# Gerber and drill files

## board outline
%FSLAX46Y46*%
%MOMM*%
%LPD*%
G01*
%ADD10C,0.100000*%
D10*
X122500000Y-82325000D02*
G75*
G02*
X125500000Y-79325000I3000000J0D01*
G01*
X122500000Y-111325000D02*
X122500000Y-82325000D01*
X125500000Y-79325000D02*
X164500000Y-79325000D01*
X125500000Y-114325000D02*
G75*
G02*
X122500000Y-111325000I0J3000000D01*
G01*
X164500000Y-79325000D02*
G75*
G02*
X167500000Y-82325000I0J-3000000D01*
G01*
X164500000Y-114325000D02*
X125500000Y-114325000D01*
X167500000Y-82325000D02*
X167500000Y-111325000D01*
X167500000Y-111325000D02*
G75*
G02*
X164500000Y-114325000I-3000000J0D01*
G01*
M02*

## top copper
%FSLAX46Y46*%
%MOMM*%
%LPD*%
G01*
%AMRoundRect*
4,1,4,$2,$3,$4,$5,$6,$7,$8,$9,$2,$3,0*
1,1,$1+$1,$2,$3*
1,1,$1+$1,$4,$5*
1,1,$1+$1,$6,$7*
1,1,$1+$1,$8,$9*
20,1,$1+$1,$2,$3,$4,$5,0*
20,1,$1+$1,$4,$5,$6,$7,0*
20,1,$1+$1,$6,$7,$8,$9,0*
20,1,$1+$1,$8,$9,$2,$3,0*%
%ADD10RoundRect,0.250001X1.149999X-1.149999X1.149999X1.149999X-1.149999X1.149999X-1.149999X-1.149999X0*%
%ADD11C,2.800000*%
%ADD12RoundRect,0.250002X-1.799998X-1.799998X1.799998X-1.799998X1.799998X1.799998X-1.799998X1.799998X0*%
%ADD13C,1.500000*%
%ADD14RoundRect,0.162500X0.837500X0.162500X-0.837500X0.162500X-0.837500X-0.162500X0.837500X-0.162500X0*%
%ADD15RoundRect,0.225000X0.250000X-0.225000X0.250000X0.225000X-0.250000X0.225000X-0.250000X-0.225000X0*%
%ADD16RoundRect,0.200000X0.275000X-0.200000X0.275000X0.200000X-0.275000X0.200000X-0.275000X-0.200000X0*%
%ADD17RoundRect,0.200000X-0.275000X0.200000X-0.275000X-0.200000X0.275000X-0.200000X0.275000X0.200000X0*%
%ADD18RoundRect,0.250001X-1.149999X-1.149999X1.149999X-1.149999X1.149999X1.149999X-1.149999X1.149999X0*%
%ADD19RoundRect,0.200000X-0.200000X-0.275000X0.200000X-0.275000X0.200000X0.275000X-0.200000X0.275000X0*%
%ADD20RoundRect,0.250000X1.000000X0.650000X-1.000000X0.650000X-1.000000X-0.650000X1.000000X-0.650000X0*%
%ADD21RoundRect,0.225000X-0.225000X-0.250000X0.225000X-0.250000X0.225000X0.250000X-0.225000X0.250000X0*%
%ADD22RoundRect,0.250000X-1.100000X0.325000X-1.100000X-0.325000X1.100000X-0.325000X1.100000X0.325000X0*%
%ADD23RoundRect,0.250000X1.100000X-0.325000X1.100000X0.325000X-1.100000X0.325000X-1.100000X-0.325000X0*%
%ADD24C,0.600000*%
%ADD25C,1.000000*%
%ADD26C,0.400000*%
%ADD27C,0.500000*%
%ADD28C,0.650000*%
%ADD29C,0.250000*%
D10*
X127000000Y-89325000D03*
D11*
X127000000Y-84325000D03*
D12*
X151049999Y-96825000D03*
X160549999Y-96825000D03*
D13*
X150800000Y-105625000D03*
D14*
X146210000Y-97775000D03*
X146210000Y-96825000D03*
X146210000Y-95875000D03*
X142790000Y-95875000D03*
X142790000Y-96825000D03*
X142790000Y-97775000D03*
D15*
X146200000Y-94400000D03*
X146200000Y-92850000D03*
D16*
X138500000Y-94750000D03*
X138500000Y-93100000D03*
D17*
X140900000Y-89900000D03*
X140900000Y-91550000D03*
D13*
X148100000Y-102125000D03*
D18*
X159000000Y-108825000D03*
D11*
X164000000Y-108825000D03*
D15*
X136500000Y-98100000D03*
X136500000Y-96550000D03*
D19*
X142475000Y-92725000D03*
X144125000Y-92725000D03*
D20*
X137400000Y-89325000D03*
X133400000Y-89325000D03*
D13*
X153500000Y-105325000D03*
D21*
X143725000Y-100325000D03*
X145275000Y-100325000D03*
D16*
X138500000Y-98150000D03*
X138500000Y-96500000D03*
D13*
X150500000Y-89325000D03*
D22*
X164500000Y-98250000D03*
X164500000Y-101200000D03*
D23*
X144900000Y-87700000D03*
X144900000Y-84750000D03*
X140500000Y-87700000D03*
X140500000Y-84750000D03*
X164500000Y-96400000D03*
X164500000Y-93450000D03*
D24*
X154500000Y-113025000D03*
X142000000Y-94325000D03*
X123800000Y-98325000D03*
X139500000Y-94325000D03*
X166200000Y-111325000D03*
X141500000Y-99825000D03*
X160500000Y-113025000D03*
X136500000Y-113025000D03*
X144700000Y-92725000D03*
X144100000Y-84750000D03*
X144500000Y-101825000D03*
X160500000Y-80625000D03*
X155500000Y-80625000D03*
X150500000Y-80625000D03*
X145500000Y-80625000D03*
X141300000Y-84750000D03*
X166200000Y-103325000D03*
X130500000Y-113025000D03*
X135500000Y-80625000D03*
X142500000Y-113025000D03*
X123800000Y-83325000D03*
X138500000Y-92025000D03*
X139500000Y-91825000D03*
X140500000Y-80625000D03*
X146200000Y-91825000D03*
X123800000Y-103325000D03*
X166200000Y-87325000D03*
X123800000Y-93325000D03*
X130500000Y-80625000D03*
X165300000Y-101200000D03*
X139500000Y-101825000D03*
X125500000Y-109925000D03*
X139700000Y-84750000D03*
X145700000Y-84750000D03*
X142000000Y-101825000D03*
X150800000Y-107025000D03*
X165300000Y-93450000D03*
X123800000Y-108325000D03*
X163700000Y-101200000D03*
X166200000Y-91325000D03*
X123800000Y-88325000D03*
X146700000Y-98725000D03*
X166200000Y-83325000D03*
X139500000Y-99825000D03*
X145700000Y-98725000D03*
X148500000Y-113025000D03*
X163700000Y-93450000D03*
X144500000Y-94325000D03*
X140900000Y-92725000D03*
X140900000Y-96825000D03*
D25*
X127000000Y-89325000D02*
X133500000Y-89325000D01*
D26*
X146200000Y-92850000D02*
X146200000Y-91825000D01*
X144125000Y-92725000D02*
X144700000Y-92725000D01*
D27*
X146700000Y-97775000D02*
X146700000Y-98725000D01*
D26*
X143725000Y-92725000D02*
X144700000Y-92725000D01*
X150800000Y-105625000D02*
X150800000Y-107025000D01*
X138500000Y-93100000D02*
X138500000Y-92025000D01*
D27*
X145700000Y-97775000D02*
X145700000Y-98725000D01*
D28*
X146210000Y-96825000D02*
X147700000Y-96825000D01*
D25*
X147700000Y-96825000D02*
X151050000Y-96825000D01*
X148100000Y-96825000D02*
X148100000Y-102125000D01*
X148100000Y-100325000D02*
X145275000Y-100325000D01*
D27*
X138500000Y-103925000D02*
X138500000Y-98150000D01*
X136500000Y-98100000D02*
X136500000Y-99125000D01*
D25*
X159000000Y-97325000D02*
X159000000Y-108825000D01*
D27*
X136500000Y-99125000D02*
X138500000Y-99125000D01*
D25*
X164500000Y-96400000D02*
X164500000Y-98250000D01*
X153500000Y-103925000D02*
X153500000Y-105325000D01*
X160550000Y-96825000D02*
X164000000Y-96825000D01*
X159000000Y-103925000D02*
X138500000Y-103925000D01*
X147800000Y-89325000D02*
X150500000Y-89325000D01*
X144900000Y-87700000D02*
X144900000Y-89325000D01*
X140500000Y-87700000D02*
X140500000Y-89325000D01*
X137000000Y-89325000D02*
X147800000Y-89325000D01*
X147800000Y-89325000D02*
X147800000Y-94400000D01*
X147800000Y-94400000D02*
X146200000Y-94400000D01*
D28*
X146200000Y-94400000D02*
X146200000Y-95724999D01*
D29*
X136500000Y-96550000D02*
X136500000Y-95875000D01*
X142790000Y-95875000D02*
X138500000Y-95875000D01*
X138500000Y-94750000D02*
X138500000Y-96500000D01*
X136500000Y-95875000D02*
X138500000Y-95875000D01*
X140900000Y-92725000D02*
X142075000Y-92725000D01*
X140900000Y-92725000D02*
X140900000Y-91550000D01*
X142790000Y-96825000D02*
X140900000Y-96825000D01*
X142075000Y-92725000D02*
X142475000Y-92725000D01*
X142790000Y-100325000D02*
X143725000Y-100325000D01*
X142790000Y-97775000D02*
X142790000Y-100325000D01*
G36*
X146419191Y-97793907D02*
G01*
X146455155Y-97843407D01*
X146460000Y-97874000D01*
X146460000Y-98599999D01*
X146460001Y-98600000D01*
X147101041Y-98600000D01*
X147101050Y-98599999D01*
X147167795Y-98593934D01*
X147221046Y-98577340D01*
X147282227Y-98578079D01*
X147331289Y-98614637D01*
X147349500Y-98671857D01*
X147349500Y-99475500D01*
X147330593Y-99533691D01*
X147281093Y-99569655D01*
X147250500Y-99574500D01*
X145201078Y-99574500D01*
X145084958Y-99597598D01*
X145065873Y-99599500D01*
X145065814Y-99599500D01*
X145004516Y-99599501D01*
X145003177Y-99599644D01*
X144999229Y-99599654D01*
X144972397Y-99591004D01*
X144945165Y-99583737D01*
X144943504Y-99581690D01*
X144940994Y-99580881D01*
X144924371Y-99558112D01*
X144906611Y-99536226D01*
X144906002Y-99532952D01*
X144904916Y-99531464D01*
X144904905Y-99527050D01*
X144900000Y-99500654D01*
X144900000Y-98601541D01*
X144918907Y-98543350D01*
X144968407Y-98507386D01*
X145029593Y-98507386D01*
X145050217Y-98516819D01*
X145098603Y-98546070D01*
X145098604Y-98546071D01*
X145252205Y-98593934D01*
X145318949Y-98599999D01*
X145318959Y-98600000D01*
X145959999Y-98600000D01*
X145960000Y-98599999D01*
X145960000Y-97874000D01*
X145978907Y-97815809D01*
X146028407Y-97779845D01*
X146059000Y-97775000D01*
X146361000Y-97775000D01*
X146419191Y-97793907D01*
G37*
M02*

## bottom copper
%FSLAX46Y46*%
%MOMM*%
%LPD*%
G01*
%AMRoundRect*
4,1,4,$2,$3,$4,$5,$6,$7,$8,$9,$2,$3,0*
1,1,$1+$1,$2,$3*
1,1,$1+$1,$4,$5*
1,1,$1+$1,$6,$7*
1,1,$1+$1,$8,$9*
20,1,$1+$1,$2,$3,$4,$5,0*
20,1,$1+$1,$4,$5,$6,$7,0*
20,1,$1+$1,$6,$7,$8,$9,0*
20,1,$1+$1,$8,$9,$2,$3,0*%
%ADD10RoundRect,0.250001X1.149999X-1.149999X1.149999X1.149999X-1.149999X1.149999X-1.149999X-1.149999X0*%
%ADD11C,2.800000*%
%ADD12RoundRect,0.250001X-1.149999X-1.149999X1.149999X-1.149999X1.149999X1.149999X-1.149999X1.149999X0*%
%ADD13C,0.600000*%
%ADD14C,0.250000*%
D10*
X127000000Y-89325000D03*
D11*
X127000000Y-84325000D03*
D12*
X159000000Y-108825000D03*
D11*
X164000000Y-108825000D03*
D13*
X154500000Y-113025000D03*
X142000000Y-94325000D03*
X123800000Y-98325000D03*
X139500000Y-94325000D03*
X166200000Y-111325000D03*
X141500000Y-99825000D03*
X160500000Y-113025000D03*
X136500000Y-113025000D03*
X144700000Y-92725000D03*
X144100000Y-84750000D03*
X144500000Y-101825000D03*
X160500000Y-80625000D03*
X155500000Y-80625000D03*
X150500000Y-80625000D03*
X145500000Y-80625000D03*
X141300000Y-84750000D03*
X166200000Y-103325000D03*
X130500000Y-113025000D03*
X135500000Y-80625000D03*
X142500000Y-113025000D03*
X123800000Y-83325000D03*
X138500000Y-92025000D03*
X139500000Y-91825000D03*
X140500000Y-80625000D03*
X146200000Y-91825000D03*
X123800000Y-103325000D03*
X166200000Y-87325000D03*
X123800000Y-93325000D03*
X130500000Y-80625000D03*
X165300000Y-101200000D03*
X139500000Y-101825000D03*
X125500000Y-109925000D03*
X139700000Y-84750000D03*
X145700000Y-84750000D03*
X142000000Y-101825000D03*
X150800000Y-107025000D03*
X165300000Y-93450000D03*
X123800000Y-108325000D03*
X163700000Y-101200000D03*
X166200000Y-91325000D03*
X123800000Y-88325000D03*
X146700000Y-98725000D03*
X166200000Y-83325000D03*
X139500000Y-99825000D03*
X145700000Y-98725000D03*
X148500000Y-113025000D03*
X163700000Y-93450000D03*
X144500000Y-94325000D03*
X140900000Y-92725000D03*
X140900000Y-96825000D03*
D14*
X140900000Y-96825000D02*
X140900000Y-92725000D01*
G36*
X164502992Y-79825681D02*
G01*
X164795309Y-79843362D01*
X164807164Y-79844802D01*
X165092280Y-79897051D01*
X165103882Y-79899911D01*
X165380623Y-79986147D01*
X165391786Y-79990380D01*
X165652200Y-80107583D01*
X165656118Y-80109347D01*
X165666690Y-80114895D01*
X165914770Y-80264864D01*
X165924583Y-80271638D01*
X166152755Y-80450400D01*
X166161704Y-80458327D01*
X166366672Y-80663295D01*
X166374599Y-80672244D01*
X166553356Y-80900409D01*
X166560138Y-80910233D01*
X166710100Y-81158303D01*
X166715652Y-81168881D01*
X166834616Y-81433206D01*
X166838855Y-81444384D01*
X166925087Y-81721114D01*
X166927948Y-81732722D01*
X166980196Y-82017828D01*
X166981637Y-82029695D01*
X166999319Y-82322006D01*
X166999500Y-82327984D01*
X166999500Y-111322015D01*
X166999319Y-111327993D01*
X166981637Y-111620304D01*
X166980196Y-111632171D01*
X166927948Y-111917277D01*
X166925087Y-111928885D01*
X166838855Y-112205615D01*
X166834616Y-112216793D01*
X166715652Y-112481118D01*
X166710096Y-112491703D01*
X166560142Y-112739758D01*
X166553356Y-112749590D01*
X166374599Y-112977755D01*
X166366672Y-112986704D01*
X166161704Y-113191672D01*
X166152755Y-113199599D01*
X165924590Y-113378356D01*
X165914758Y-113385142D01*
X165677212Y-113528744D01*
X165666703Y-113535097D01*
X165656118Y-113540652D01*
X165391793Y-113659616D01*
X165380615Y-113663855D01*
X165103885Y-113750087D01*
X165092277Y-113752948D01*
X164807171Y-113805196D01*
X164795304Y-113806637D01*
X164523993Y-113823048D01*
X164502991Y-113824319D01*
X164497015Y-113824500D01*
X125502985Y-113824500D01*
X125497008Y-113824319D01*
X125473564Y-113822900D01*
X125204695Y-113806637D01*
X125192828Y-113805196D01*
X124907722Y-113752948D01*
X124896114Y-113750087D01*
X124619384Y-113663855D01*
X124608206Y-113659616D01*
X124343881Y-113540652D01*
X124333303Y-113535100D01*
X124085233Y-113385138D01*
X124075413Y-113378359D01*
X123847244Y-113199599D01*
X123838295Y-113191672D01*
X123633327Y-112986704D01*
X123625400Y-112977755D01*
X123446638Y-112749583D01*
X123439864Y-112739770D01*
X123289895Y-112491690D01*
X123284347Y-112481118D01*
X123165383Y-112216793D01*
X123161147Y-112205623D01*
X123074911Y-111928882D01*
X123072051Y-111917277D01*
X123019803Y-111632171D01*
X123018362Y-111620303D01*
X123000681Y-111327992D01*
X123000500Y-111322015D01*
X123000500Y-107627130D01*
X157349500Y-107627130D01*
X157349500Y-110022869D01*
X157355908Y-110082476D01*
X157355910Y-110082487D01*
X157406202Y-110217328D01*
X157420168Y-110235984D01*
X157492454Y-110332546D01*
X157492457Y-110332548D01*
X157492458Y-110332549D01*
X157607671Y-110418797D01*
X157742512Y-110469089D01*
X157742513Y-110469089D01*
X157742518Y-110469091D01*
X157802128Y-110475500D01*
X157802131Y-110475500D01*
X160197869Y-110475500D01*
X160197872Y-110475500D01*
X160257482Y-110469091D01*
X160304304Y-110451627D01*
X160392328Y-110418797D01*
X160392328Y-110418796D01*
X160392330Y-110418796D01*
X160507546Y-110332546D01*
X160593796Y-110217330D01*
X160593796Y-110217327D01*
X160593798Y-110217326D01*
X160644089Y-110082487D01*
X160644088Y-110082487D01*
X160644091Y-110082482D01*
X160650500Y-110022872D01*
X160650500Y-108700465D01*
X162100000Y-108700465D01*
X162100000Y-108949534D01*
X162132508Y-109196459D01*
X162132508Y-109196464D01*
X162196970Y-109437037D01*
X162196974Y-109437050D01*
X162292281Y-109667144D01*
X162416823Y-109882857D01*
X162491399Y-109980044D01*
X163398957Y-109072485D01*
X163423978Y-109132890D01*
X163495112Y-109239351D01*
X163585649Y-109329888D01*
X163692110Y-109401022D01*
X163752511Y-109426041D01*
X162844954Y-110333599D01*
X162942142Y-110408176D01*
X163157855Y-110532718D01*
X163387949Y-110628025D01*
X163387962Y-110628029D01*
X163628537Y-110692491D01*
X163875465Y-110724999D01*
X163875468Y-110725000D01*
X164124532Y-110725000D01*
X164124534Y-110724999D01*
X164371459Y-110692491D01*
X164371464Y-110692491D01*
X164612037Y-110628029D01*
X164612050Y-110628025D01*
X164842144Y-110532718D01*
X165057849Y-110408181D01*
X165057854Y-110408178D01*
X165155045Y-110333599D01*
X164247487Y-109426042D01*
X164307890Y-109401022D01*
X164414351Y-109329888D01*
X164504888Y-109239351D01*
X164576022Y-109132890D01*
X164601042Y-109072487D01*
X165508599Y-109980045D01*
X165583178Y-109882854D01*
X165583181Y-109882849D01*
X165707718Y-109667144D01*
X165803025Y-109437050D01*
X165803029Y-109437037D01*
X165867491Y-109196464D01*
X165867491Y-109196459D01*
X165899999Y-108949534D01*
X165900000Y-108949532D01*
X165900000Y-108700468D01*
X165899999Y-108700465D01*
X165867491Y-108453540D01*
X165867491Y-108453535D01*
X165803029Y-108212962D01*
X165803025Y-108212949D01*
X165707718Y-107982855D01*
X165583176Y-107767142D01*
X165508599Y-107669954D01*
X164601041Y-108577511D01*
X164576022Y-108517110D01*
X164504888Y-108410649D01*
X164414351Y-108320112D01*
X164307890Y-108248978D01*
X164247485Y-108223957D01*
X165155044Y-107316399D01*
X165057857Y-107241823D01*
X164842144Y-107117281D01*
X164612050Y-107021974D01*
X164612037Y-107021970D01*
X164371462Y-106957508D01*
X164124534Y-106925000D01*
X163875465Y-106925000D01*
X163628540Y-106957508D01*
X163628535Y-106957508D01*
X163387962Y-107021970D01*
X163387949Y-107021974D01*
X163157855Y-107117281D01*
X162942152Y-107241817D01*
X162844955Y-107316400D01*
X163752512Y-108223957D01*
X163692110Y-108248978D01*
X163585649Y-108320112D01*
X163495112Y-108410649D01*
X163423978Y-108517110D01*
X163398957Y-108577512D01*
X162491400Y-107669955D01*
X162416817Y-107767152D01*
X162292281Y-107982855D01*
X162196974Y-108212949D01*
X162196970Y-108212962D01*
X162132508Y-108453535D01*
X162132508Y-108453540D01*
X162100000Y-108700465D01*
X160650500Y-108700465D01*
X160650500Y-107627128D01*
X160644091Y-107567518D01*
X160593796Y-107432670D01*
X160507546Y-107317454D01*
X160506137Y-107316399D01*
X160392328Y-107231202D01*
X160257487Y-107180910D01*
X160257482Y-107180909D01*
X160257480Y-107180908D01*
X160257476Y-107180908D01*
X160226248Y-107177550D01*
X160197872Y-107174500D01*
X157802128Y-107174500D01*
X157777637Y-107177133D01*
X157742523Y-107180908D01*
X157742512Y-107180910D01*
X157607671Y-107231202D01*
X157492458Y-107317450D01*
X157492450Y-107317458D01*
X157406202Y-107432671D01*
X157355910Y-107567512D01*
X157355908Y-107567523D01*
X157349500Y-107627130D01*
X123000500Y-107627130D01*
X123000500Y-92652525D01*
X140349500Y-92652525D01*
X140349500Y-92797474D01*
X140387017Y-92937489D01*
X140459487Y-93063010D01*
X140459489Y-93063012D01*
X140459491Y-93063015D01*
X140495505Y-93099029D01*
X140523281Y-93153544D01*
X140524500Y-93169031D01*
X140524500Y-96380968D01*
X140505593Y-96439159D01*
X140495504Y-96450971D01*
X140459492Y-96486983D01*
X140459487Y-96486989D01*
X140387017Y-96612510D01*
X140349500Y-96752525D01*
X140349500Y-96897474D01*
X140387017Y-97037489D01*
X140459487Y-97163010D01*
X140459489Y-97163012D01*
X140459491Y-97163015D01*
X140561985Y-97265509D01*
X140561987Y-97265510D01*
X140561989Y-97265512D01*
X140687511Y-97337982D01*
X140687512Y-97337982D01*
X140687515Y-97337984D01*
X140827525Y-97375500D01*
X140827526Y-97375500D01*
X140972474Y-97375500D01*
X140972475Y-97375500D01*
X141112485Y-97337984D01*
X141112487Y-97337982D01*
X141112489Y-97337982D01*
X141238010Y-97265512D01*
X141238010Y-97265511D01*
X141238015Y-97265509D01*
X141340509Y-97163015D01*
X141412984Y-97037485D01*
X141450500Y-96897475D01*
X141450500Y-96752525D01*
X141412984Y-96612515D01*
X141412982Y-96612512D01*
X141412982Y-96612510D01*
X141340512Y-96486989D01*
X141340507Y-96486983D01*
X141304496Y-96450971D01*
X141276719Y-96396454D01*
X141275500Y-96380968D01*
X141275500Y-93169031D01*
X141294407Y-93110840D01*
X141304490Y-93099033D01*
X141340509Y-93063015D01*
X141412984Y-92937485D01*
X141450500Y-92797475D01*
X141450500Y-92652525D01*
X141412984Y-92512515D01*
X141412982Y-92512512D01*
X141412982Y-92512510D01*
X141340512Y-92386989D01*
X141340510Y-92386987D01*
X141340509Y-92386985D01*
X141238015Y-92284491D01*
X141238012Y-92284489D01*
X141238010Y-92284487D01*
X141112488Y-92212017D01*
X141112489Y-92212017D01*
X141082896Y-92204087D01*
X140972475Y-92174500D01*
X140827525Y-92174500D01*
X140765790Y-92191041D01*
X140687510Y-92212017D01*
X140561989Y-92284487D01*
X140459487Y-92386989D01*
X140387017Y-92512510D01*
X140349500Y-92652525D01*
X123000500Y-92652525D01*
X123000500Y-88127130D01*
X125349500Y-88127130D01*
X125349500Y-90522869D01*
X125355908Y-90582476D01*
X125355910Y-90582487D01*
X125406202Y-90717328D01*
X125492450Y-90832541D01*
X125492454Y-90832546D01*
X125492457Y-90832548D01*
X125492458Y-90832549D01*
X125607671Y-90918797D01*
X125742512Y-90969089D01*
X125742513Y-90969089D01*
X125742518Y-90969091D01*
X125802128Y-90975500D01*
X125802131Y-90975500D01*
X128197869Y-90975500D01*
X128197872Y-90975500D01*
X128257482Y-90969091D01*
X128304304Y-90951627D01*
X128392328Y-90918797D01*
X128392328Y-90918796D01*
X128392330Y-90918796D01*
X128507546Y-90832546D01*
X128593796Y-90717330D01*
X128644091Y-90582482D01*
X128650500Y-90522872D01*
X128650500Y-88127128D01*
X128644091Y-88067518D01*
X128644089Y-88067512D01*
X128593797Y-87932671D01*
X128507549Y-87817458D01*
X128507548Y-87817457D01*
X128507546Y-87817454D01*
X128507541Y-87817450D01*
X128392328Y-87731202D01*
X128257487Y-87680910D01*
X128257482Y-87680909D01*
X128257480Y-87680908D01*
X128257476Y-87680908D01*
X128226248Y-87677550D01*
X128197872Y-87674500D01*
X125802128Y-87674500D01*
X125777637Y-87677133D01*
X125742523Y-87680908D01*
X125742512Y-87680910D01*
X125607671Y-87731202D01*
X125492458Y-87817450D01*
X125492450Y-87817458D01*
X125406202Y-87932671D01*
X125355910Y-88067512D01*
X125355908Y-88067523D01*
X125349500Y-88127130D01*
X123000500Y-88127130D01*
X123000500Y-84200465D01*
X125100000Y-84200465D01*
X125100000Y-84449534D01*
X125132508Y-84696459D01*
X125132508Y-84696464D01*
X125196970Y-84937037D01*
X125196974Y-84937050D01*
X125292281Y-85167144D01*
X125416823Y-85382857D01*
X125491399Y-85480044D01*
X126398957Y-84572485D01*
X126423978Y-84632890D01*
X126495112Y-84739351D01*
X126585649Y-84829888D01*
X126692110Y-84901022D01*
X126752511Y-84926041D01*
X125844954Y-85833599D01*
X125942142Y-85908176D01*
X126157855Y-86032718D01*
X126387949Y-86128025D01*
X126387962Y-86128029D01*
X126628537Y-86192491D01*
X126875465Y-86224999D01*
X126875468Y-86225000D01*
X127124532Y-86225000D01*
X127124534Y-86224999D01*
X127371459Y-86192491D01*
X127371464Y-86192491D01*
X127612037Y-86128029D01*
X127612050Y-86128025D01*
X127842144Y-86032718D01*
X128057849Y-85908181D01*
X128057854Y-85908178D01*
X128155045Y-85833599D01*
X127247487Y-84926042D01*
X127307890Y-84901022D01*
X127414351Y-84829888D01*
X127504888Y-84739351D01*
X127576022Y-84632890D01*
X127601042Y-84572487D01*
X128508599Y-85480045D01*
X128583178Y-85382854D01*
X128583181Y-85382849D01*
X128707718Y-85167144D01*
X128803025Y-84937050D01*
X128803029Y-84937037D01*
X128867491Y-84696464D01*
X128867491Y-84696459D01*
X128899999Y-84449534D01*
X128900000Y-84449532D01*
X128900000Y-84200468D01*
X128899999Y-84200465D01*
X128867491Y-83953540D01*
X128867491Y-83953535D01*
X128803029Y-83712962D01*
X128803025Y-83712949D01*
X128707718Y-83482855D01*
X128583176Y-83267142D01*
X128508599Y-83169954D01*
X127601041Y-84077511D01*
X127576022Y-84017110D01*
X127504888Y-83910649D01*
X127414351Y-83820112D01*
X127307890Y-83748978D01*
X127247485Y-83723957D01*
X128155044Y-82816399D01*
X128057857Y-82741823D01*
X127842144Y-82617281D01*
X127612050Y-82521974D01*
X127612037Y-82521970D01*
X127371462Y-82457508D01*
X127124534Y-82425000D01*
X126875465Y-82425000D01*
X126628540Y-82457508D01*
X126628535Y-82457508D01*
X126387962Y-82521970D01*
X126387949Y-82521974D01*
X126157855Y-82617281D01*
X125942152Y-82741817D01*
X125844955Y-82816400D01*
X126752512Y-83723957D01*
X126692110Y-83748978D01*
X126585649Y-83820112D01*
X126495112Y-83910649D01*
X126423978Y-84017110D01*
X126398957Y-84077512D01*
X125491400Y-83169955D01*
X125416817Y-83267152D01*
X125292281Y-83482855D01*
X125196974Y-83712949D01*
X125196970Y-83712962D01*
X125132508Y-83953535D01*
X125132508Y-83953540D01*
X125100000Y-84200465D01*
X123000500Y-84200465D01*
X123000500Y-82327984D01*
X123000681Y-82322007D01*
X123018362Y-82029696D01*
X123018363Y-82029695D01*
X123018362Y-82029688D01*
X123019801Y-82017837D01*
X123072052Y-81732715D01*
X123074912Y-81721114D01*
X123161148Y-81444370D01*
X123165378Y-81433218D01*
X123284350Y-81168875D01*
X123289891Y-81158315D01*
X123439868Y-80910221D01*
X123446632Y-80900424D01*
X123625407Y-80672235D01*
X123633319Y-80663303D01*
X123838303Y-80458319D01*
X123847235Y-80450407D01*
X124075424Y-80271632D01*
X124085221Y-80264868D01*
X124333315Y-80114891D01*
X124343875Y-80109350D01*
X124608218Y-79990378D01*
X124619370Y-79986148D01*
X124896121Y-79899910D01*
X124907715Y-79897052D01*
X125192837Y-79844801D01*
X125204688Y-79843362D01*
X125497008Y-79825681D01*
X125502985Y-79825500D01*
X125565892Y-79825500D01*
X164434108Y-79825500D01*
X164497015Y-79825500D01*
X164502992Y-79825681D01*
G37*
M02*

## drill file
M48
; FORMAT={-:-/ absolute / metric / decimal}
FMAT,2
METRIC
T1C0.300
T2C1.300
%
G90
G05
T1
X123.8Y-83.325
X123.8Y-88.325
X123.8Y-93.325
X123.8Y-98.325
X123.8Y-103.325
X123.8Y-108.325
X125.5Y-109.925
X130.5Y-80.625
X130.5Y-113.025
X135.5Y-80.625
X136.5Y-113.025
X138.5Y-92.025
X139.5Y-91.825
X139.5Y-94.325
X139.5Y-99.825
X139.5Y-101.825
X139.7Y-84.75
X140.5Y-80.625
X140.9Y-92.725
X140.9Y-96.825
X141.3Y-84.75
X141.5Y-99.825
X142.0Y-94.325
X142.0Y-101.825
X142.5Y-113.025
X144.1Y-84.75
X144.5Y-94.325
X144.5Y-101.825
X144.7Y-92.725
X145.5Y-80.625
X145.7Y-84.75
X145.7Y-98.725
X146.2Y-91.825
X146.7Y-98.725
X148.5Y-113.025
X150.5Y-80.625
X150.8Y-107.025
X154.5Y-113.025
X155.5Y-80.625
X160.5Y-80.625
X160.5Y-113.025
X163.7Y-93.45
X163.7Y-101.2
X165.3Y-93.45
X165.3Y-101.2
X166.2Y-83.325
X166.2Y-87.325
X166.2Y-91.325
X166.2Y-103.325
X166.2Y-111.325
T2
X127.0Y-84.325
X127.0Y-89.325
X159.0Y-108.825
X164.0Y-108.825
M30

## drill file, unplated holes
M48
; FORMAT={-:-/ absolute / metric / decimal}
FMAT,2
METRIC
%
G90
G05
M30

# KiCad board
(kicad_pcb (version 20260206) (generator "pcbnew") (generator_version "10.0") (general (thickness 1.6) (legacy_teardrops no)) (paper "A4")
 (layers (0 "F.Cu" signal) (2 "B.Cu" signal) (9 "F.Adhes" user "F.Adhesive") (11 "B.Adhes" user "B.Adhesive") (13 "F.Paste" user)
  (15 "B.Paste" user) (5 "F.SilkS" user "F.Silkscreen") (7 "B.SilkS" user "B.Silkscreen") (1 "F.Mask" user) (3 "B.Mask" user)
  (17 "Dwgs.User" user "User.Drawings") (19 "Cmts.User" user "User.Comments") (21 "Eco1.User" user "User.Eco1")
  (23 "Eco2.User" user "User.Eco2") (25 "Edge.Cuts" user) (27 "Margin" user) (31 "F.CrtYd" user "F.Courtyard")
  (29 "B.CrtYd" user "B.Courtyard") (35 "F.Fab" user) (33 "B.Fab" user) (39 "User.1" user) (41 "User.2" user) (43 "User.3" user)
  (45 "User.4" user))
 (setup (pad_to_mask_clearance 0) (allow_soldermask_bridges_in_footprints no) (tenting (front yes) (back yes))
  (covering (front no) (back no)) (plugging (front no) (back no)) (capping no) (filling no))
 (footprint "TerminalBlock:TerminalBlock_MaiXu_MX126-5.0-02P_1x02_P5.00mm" (layer "F.Cu") (at 127 89.325 90)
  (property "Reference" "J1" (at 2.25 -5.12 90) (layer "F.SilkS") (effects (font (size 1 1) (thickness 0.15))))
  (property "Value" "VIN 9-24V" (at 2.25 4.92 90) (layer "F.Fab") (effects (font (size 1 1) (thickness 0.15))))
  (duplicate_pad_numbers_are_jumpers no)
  (pad "1" thru_hole roundrect (at 0 0 90) (size 2.8 2.8) (drill 1.3) (layers "*.Cu" "*.Mask") (remove_unused_layers no)
   (roundrect_rratio 0.089286) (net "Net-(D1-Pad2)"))
  (pad "2" thru_hole circle (at 5 0 90) (size 2.8 2.8) (drill 1.3) (layers "*.Cu" "*.Mask") (remove_unused_layers no) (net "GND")))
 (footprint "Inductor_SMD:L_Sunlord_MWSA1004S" (layer "F.Cu") (at 155.799999 96.825)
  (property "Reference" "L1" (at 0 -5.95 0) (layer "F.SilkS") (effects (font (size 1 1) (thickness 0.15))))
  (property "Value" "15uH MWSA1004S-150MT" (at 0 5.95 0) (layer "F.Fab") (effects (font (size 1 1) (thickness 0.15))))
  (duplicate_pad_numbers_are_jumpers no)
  (pad "1" smd roundrect (at -4.75 0) (size 4.1 4.1) (layers "F.Cu" "F.Mask" "F.Paste") (roundrect_rratio 0.060976) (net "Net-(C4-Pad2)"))
  (pad "2" smd roundrect (at 4.75 0) (size 4.1 4.1) (layers "F.Cu" "F.Mask" "F.Paste") (roundrect_rratio 0.060976) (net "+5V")))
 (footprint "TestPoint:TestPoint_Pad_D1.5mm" (layer "F.Cu") (at 150.8 105.625)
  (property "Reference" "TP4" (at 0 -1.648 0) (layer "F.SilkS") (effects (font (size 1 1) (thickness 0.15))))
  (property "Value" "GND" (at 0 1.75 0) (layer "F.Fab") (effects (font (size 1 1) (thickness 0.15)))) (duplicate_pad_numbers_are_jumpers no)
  (pad "1" smd circle (at 0 0) (size 1.5 1.5) (layers "F.Cu" "F.Mask") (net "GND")))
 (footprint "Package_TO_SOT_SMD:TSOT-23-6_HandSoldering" (layer "F.Cu") (at 144.5 96.825 180)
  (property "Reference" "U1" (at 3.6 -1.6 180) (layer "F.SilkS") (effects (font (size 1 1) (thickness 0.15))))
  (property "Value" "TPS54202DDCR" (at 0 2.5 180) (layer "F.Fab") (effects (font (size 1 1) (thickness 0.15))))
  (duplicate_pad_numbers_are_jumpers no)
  (pad "1" smd roundrect (at -1.71 -0.95 180) (size 2 0.65) (layers "F.Cu" "F.Mask" "F.Paste") (roundrect_rratio 0.25) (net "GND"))
  (pad "2" smd roundrect (at -1.71 0 180) (size 2 0.65) (layers "F.Cu" "F.Mask" "F.Paste") (roundrect_rratio 0.25) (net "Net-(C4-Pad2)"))
  (pad "3" smd roundrect (at -1.71 0.95 180) (size 2 0.65) (layers "F.Cu" "F.Mask" "F.Paste") (roundrect_rratio 0.25) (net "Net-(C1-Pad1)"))
  (pad "4" smd roundrect (at 1.71 0.95 180) (size 2 0.65) (layers "F.Cu" "F.Mask" "F.Paste") (roundrect_rratio 0.25) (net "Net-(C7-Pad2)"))
  (pad "5" smd roundrect (at 1.71 0 180) (size 2 0.65) (layers "F.Cu" "F.Mask" "F.Paste") (roundrect_rratio 0.25) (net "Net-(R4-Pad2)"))
  (pad "6" smd roundrect (at 1.71 -0.95 180) (size 2 0.65) (layers "F.Cu" "F.Mask" "F.Paste") (roundrect_rratio 0.25) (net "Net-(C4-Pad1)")))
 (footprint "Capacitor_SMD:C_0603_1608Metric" (layer "F.Cu") (at 146.2 93.625 90)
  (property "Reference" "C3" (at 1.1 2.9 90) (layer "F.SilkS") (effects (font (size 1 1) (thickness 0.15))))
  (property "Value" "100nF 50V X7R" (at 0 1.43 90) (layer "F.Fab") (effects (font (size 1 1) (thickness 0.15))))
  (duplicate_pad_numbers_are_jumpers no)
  (pad "1" smd roundrect (at -0.775 0 90) (size 0.9 0.95) (layers "F.Cu" "F.Mask" "F.Paste") (roundrect_rratio 0.25) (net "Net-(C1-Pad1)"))
  (pad "2" smd roundrect (at 0.775 0 90) (size 0.9 0.95) (layers "F.Cu" "F.Mask" "F.Paste") (roundrect_rratio 0.25) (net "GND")))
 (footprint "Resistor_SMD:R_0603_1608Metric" (layer "F.Cu") (at 138.5 93.925 90)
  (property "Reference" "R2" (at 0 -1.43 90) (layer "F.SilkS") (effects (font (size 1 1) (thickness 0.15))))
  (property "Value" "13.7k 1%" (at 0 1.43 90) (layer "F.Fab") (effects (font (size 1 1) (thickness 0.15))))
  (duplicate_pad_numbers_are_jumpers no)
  (pad "1" smd roundrect (at -0.825 0 90) (size 0.8 0.95) (layers "F.Cu" "F.Mask" "F.Paste") (roundrect_rratio 0.25) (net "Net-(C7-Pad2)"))
  (pad "2" smd roundrect (at 0.825 0 90) (size 0.8 0.95) (layers "F.Cu" "F.Mask" "F.Paste") (roundrect_rratio 0.25) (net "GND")))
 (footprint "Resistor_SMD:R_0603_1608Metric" (layer "F.Cu") (at 140.9 90.725 -90)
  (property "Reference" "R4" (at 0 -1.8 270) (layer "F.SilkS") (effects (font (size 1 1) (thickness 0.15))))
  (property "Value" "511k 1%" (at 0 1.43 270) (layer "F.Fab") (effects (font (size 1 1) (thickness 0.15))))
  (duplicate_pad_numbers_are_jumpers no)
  (pad "1" smd roundrect (at -0.825 0 270) (size 0.8 0.95) (layers "F.Cu" "F.Mask" "F.Paste") (roundrect_rratio 0.25) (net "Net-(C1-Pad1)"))
  (pad "2" smd roundrect (at 0.825 0 270) (size 0.8 0.95) (layers "F.Cu" "F.Mask" "F.Paste") (roundrect_rratio 0.25) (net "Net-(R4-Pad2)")))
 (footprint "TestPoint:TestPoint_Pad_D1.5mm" (layer "F.Cu") (at 148.1 102.125)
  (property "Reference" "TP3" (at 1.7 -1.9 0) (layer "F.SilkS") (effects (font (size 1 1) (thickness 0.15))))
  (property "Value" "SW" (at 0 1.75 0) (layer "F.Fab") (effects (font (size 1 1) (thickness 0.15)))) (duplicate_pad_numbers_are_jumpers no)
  (pad "1" smd circle (at 0 0) (size 1.5 1.5) (layers "F.Cu" "F.Mask") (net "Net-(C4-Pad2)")))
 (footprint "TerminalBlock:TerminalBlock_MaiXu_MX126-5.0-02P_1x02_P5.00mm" (layer "F.Cu") (at 159 108.825)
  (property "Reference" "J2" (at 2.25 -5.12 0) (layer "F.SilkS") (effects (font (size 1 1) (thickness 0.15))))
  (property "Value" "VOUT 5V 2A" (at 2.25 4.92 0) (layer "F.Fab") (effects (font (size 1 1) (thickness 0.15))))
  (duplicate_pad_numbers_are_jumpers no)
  (pad "1" thru_hole roundrect (at 0 0) (size 2.8 2.8) (drill 1.3) (layers "*.Cu" "*.Mask") (remove_unused_layers no)
   (roundrect_rratio 0.089286) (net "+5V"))
  (pad "2" thru_hole circle (at 5 0) (size 2.8 2.8) (drill 1.3) (layers "*.Cu" "*.Mask") (remove_unused_layers no) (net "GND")))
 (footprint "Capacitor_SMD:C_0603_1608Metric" (layer "F.Cu") (at 136.5 97.325 90)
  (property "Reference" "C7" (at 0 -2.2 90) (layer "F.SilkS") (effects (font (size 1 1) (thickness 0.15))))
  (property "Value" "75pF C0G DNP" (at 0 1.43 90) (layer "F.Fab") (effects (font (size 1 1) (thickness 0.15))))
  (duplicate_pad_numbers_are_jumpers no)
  (pad "1" smd roundrect (at -0.775 0 90) (size 0.9 0.95) (layers "F.Cu" "F.Mask" "F.Paste") (roundrect_rratio 0.25) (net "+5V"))
  (pad "2" smd roundrect (at 0.775 0 90) (size 0.9 0.95) (layers "F.Cu" "F.Mask" "F.Paste") (roundrect_rratio 0.25) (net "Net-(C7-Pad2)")))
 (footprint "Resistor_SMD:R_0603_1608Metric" (layer "F.Cu") (at 143.3 92.725)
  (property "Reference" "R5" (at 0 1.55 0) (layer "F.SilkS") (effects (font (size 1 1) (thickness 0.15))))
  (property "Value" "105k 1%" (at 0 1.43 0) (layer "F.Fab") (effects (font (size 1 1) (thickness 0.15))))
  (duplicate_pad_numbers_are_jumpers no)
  (pad "1" smd roundrect (at -0.825 0) (size 0.8 0.95) (layers "F.Cu" "F.Mask" "F.Paste") (roundrect_rratio 0.25) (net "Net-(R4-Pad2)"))
  (pad "2" smd roundrect (at 0.825 0) (size 0.8 0.95) (layers "F.Cu" "F.Mask" "F.Paste") (roundrect_rratio 0.25) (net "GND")))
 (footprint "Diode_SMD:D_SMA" (layer "F.Cu") (at 135.4 89.325 180)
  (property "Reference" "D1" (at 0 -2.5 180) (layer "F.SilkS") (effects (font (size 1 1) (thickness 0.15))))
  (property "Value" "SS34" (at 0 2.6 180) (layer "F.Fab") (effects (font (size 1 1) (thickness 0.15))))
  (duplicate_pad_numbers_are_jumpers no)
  (pad "1" smd roundrect (at -2 0 180) (size 2.5 1.8) (layers "F.Cu" "F.Mask" "F.Paste") (roundrect_rratio 0.1388888889)
   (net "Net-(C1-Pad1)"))
  (pad "2" smd roundrect (at 2 0 180) (size 2.5 1.8) (layers "F.Cu" "F.Mask" "F.Paste") (roundrect_rratio 0.1388888889)
   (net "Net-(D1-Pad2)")))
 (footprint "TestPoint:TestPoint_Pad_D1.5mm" (layer "F.Cu") (at 153.5 105.325)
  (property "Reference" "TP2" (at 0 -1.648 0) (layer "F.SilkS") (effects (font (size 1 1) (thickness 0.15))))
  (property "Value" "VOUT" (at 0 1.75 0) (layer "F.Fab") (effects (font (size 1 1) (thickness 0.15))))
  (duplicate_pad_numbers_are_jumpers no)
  (pad "1" smd circle (at 0 0) (size 1.5 1.5) (layers "F.Cu" "F.Mask") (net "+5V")))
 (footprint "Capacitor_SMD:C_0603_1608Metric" (layer "F.Cu") (at 144.5 100.325)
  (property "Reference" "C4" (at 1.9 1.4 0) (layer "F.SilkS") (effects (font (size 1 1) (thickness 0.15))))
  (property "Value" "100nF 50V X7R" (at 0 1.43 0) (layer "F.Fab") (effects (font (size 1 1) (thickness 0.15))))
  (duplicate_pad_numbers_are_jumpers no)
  (pad "1" smd roundrect (at -0.775 0) (size 0.9 0.95) (layers "F.Cu" "F.Mask" "F.Paste") (roundrect_rratio 0.25) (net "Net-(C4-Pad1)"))
  (pad "2" smd roundrect (at 0.775 0) (size 0.9 0.95) (layers "F.Cu" "F.Mask" "F.Paste") (roundrect_rratio 0.25) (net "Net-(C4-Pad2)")))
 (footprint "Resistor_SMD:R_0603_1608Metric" (layer "F.Cu") (at 138.5 97.325 90)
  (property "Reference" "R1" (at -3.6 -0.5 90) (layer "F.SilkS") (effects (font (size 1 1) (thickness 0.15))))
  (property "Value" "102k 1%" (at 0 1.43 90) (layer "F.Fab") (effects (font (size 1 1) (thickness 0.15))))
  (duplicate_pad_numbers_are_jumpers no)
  (pad "1" smd roundrect (at -0.825 0 90) (size 0.8 0.95) (layers "F.Cu" "F.Mask" "F.Paste") (roundrect_rratio 0.25) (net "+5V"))
  (pad "2" smd roundrect (at 0.825 0 90) (size 0.8 0.95) (layers "F.Cu" "F.Mask" "F.Paste") (roundrect_rratio 0.25) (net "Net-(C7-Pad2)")))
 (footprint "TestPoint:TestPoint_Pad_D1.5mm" (layer "F.Cu") (at 150.5 89.325)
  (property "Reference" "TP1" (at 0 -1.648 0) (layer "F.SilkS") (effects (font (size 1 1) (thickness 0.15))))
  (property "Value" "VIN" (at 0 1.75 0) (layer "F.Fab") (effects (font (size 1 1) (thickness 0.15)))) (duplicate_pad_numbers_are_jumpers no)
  (pad "1" smd circle (at 0 0) (size 1.5 1.5) (layers "F.Cu" "F.Mask") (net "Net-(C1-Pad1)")))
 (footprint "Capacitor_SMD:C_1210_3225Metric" (layer "F.Cu") (at 164.5 99.725 -90)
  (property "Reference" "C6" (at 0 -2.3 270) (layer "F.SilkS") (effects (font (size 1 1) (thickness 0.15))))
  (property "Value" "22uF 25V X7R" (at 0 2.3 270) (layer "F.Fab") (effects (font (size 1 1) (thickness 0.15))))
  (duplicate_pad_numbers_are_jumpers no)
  (pad "1" smd roundrect (at -1.475 0 270) (size 1.15 2.7) (layers "F.Cu" "F.Mask" "F.Paste") (roundrect_rratio 0.217391) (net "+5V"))
  (pad "2" smd roundrect (at 1.475 0 270) (size 1.15 2.7) (layers "F.Cu" "F.Mask" "F.Paste") (roundrect_rratio 0.217391) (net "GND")))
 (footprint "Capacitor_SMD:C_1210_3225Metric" (layer "F.Cu") (at 144.9 86.225 90)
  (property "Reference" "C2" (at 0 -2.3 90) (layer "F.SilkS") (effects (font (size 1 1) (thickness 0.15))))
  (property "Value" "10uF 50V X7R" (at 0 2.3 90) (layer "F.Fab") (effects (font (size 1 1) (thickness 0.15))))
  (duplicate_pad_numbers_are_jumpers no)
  (pad "1" smd roundrect (at -1.475 0 90) (size 1.15 2.7) (layers "F.Cu" "F.Mask" "F.Paste") (roundrect_rratio 0.217391)
   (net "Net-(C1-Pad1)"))
  (pad "2" smd roundrect (at 1.475 0 90) (size 1.15 2.7) (layers "F.Cu" "F.Mask" "F.Paste") (roundrect_rratio 0.217391) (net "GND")))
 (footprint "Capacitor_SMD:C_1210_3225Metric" (layer "F.Cu") (at 140.5 86.225 90)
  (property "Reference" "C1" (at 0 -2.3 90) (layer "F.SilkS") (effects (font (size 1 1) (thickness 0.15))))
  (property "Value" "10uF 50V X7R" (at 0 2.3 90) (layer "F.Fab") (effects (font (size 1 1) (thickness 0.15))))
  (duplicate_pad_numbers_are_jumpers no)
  (pad "1" smd roundrect (at -1.475 0 90) (size 1.15 2.7) (layers "F.Cu" "F.Mask" "F.Paste") (roundrect_rratio 0.217391)
   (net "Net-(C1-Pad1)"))
  (pad "2" smd roundrect (at 1.475 0 90) (size 1.15 2.7) (layers "F.Cu" "F.Mask" "F.Paste") (roundrect_rratio 0.217391) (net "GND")))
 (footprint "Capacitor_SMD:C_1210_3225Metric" (layer "F.Cu") (at 164.5 94.925 90)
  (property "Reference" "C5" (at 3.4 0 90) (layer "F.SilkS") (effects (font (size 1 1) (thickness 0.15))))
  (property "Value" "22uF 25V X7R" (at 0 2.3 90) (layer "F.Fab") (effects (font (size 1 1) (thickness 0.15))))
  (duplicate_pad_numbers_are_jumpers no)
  (pad "1" smd roundrect (at -1.475 0 90) (size 1.15 2.7) (layers "F.Cu" "F.Mask" "F.Paste") (roundrect_rratio 0.217391) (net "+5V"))
  (pad "2" smd roundrect (at 1.475 0 90) (size 1.15 2.7) (layers "F.Cu" "F.Mask" "F.Paste") (roundrect_rratio 0.217391) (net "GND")))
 (gr_arc (start 122.5 82.325) (mid 123.37868 80.20368) (end 125.5 79.325) (stroke (width 0.1) (type default)) (layer "Edge.Cuts"))
 (gr_line (start 122.5 111.325) (end 122.5 82.325) (stroke (width 0.1) (type default)) (layer "Edge.Cuts"))
 (gr_line (start 125.5 79.325) (end 164.5 79.325) (stroke (width 0.1) (type default)) (layer "Edge.Cuts"))
 (gr_arc (start 125.5 114.325) (mid 123.37868 113.44632) (end 122.5 111.325) (stroke (width 0.1) (type default)) (layer "Edge.Cuts"))
 (gr_arc (start 164.5 79.325) (mid 166.62132 80.20368) (end 167.5 82.325) (stroke (width 0.1) (type default)) (layer "Edge.Cuts"))
 (gr_line (start 164.5 114.325) (end 125.5 114.325) (stroke (width 0.1) (type default)) (layer "Edge.Cuts"))
 (gr_line (start 167.5 82.325) (end 167.5 111.325) (stroke (width 0.1) (type default)) (layer "Edge.Cuts"))
 (gr_arc (start 167.5 111.325) (mid 166.62132 113.44632) (end 164.5 114.325) (stroke (width 0.1) (type default)) (layer "Edge.Cuts"))
 (segment (start 127 89.325) (end 133.5 89.325) (width 1) (layer "F.Cu") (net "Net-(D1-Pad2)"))
 (segment (start 146.2 92.85) (end 146.2 91.825) (width 0.4) (layer "F.Cu") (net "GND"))
 (segment (start 144.125 92.725) (end 144.7 92.725) (width 0.4) (layer "F.Cu") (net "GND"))
 (segment (start 146.7 97.775) (end 146.7 98.725) (width 0.5) (layer "F.Cu") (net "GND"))
 (segment (start 143.725 92.725) (end 144.7 92.725) (width 0.4) (layer "F.Cu") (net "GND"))
 (segment (start 150.8 105.625) (end 150.8 107.025) (width 0.4) (layer "F.Cu") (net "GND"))
 (segment (start 138.5 93.1) (end 138.5 92.025) (width 0.4) (layer "F.Cu") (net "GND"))
 (segment (start 145.7 97.775) (end 145.7 98.725) (width 0.5) (layer "F.Cu") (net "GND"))
 (via (at 154.5 113.025) (size 0.6) (drill 0.3) (layers "F.Cu" "B.Cu") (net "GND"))
 (via (at 142 94.325) (size 0.6) (drill 0.3) (layers "F.Cu" "B.Cu") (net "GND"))
 (via (at 123.8 98.325) (size 0.6) (drill 0.3) (layers "F.Cu" "B.Cu") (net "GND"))
 (via (at 139.5 94.325) (size 0.6) (drill 0.3) (layers "F.Cu" "B.Cu") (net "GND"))
 (via (at 166.2 111.325) (size 0.6) (drill 0.3) (layers "F.Cu" "B.Cu") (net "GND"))
 (via (at 141.5 99.825) (size 0.6) (drill 0.3) (layers "F.Cu" "B.Cu") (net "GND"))
 (via (at 160.5 113.025) (size 0.6) (drill 0.3) (layers "F.Cu" "B.Cu") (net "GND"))
 (via (at 136.5 113.025) (size 0.6) (drill 0.3) (layers "F.Cu" "B.Cu") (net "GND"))
 (via (at 144.7 92.725) (size 0.6) (drill 0.3) (layers "F.Cu" "B.Cu") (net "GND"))
 (via (at 144.1 84.75) (size 0.6) (drill 0.3) (layers "F.Cu" "B.Cu") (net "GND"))
 (via (at 144.5 101.825) (size 0.6) (drill 0.3) (layers "F.Cu" "B.Cu") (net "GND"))
 (via (at 160.5 80.625) (size 0.6) (drill 0.3) (layers "F.Cu" "B.Cu") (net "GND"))
 (via (at 155.5 80.625) (size 0.6) (drill 0.3) (layers "F.Cu" "B.Cu") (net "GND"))
 (via (at 150.5 80.625) (size 0.6) (drill 0.3) (layers "F.Cu" "B.Cu") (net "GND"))
 (via (at 145.5 80.625) (size 0.6) (drill 0.3) (layers "F.Cu" "B.Cu") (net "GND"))
 (via (at 141.3 84.75) (size 0.6) (drill 0.3) (layers "F.Cu" "B.Cu") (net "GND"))
 (via (at 166.2 103.325) (size 0.6) (drill 0.3) (layers "F.Cu" "B.Cu") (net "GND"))
 (via (at 130.5 113.025) (size 0.6) (drill 0.3) (layers "F.Cu" "B.Cu") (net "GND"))
 (via (at 135.5 80.625) (size 0.6) (drill 0.3) (layers "F.Cu" "B.Cu") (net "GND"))
 (via (at 142.5 113.025) (size 0.6) (drill 0.3) (layers "F.Cu" "B.Cu") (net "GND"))
 (via (at 123.8 83.325) (size 0.6) (drill 0.3) (layers "F.Cu" "B.Cu") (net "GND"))
 (via (at 138.5 92.025) (size 0.6) (drill 0.3) (layers "F.Cu" "B.Cu") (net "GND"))
 (via (at 139.5 91.825) (size 0.6) (drill 0.3) (layers "F.Cu" "B.Cu") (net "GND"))
 (via (at 140.5 80.625) (size 0.6) (drill 0.3) (layers "F.Cu" "B.Cu") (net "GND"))
 (via (at 146.2 91.825) (size 0.6) (drill 0.3) (layers "F.Cu" "B.Cu") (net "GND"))
 (via (at 123.8 103.325) (size 0.6) (drill 0.3) (layers "F.Cu" "B.Cu") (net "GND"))
 (via (at 166.2 87.325) (size 0.6) (drill 0.3) (layers "F.Cu" "B.Cu") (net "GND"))
 (via (at 123.8 93.325) (size 0.6) (drill 0.3) (layers "F.Cu" "B.Cu") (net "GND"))
 (via (at 130.5 80.625) (size 0.6) (drill 0.3) (layers "F.Cu" "B.Cu") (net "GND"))
 (via (at 165.3 101.2) (size 0.6) (drill 0.3) (layers "F.Cu" "B.Cu") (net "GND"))
 (via (at 139.5 101.825) (size 0.6) (drill 0.3) (layers "F.Cu" "B.Cu") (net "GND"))
 (via (at 125.5 109.925) (size 0.6) (drill 0.3) (layers "F.Cu" "B.Cu") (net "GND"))
 (via (at 139.7 84.75) (size 0.6) (drill 0.3) (layers "F.Cu" "B.Cu") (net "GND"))
 (via (at 145.7 84.75) (size 0.6) (drill 0.3) (layers "F.Cu" "B.Cu") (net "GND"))
 (via (at 142 101.825) (size 0.6) (drill 0.3) (layers "F.Cu" "B.Cu") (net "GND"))
 (via (at 150.8 107.025) (size 0.6) (drill 0.3) (layers "F.Cu" "B.Cu") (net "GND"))
 (via (at 165.3 93.45) (size 0.6) (drill 0.3) (layers "F.Cu" "B.Cu") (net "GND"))
 (via (at 123.8 108.325) (size 0.6) (drill 0.3) (layers "F.Cu" "B.Cu") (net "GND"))
 (via (at 163.7 101.2) (size 0.6) (drill 0.3) (layers "F.Cu" "B.Cu") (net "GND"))
 (via (at 166.2 91.325) (size 0.6) (drill 0.3) (layers "F.Cu" "B.Cu") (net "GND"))
 (via (at 123.8 88.325) (size 0.6) (drill 0.3) (layers "F.Cu" "B.Cu") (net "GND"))
 (via (at 146.7 98.725) (size 0.6) (drill 0.3) (layers "F.Cu" "B.Cu") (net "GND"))
 (via (at 166.2 83.325) (size 0.6) (drill 0.3) (layers "F.Cu" "B.Cu") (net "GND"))
 (via (at 139.5 99.825) (size 0.6) (drill 0.3) (layers "F.Cu" "B.Cu") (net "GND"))
 (via (at 145.7 98.725) (size 0.6) (drill 0.3) (layers "F.Cu" "B.Cu") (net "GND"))
 (via (at 148.5 113.025) (size 0.6) (drill 0.3) (layers "F.Cu" "B.Cu") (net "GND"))
 (via (at 163.7 93.45) (size 0.6) (drill 0.3) (layers "F.Cu" "B.Cu") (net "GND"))
 (via (at 144.5 94.325) (size 0.6) (drill 0.3) (layers "F.Cu" "B.Cu") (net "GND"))
 (segment (start 146.21 96.825) (end 147.7 96.825) (width 0.65) (layer "F.Cu") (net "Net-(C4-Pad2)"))
 (segment (start 147.7 96.825) (end 151.05 96.825) (width 1) (layer "F.Cu") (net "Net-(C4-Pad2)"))
 (segment (start 148.1 96.825) (end 148.1 102.125) (width 1) (layer "F.Cu") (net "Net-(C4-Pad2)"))
 (segment (start 148.1 100.325) (end 145.275 100.325) (width 1) (layer "F.Cu") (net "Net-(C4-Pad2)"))
 (segment (start 138.5 103.925) (end 138.5 98.15) (width 0.5) (layer "F.Cu") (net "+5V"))
 (segment (start 136.5 98.1) (end 136.5 99.125) (width 0.5) (layer "F.Cu") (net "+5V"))
 (segment (start 159 97.325) (end 159 108.825) (width 1) (layer "F.Cu") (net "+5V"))
 (segment (start 136.5 99.125) (end 138.5 99.125) (width 0.5) (layer "F.Cu") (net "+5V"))
 (segment (start 164.5 96.4) (end 164.5 98.25) (width 1) (layer "F.Cu") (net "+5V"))
 (segment (start 153.5 103.925) (end 153.5 105.325) (width 1) (layer "F.Cu") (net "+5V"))
 (segment (start 160.55 96.825) (end 164 96.825) (width 1) (layer "F.Cu") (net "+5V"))
 (segment (start 159 103.925) (end 138.5 103.925) (width 1) (layer "F.Cu") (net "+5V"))
 (segment (start 147.8 89.325) (end 150.5 89.325) (width 1) (layer "F.Cu") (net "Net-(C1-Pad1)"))
 (segment (start 144.9 87.7) (end 144.9 89.325) (width 1) (layer "F.Cu") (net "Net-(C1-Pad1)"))
 (segment (start 140.5 87.7) (end 140.5 89.325) (width 1) (layer "F.Cu") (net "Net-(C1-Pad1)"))
 (segment (start 137 89.325) (end 147.8 89.325) (width 1) (layer "F.Cu") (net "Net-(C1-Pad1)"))
 (segment (start 147.8 89.325) (end 147.8 94.4) (width 1) (layer "F.Cu") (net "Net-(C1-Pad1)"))
 (segment (start 147.8 94.4) (end 146.2 94.4) (width 1) (layer "F.Cu") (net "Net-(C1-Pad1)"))
 (segment (start 146.2 94.4) (end 146.2 95.724999) (width 0.65) (layer "F.Cu") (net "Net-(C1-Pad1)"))
 (segment (start 136.5 96.55) (end 136.5 95.875) (width 0.25) (layer "F.Cu") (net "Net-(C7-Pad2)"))
 (segment (start 142.79 95.875) (end 138.5 95.875) (width 0.25) (layer "F.Cu") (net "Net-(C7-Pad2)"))
 (segment (start 138.5 94.75) (end 138.5 96.5) (width 0.25) (layer "F.Cu") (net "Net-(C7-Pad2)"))
 (segment (start 136.5 95.875) (end 138.5 95.875) (width 0.25) (layer "F.Cu") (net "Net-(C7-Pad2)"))
 (segment (start 140.9 92.725) (end 142.075 92.725) (width 0.25) (layer "F.Cu") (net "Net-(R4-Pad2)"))
 (segment (start 140.9 92.725) (end 140.9 91.55) (width 0.25) (layer "F.Cu") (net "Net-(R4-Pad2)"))
 (segment (start 142.79 96.825) (end 140.9 96.825) (width 0.25) (layer "F.Cu") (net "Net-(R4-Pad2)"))
 (segment (start 142.075 92.725) (end 142.475 92.725) (width 0.25) (layer "F.Cu") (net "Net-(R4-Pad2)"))
 (via (at 140.9 92.725) (size 0.6) (drill 0.3) (layers "F.Cu" "B.Cu") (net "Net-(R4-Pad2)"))
 (via (at 140.9 96.825) (size 0.6) (drill 0.3) (layers "F.Cu" "B.Cu") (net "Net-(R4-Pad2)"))
 (segment (start 140.9 96.825) (end 140.9 92.725) (width 0.25) (layer "B.Cu") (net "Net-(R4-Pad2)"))
 (segment (start 142.79 100.325) (end 143.725 100.325) (width 0.25) (layer "F.Cu") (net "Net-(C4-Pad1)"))
 (segment (start 142.79 97.775) (end 142.79 100.325) (width 0.25) (layer "F.Cu") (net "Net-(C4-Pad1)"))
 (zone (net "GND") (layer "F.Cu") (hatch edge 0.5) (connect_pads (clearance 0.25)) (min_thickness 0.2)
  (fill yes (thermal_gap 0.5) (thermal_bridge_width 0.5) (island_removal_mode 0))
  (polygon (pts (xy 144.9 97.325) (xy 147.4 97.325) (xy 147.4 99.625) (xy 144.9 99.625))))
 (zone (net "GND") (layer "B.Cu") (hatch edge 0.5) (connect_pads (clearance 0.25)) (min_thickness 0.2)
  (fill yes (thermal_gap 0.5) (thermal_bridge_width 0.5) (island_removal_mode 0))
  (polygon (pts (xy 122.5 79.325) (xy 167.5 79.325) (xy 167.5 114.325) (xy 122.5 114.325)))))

